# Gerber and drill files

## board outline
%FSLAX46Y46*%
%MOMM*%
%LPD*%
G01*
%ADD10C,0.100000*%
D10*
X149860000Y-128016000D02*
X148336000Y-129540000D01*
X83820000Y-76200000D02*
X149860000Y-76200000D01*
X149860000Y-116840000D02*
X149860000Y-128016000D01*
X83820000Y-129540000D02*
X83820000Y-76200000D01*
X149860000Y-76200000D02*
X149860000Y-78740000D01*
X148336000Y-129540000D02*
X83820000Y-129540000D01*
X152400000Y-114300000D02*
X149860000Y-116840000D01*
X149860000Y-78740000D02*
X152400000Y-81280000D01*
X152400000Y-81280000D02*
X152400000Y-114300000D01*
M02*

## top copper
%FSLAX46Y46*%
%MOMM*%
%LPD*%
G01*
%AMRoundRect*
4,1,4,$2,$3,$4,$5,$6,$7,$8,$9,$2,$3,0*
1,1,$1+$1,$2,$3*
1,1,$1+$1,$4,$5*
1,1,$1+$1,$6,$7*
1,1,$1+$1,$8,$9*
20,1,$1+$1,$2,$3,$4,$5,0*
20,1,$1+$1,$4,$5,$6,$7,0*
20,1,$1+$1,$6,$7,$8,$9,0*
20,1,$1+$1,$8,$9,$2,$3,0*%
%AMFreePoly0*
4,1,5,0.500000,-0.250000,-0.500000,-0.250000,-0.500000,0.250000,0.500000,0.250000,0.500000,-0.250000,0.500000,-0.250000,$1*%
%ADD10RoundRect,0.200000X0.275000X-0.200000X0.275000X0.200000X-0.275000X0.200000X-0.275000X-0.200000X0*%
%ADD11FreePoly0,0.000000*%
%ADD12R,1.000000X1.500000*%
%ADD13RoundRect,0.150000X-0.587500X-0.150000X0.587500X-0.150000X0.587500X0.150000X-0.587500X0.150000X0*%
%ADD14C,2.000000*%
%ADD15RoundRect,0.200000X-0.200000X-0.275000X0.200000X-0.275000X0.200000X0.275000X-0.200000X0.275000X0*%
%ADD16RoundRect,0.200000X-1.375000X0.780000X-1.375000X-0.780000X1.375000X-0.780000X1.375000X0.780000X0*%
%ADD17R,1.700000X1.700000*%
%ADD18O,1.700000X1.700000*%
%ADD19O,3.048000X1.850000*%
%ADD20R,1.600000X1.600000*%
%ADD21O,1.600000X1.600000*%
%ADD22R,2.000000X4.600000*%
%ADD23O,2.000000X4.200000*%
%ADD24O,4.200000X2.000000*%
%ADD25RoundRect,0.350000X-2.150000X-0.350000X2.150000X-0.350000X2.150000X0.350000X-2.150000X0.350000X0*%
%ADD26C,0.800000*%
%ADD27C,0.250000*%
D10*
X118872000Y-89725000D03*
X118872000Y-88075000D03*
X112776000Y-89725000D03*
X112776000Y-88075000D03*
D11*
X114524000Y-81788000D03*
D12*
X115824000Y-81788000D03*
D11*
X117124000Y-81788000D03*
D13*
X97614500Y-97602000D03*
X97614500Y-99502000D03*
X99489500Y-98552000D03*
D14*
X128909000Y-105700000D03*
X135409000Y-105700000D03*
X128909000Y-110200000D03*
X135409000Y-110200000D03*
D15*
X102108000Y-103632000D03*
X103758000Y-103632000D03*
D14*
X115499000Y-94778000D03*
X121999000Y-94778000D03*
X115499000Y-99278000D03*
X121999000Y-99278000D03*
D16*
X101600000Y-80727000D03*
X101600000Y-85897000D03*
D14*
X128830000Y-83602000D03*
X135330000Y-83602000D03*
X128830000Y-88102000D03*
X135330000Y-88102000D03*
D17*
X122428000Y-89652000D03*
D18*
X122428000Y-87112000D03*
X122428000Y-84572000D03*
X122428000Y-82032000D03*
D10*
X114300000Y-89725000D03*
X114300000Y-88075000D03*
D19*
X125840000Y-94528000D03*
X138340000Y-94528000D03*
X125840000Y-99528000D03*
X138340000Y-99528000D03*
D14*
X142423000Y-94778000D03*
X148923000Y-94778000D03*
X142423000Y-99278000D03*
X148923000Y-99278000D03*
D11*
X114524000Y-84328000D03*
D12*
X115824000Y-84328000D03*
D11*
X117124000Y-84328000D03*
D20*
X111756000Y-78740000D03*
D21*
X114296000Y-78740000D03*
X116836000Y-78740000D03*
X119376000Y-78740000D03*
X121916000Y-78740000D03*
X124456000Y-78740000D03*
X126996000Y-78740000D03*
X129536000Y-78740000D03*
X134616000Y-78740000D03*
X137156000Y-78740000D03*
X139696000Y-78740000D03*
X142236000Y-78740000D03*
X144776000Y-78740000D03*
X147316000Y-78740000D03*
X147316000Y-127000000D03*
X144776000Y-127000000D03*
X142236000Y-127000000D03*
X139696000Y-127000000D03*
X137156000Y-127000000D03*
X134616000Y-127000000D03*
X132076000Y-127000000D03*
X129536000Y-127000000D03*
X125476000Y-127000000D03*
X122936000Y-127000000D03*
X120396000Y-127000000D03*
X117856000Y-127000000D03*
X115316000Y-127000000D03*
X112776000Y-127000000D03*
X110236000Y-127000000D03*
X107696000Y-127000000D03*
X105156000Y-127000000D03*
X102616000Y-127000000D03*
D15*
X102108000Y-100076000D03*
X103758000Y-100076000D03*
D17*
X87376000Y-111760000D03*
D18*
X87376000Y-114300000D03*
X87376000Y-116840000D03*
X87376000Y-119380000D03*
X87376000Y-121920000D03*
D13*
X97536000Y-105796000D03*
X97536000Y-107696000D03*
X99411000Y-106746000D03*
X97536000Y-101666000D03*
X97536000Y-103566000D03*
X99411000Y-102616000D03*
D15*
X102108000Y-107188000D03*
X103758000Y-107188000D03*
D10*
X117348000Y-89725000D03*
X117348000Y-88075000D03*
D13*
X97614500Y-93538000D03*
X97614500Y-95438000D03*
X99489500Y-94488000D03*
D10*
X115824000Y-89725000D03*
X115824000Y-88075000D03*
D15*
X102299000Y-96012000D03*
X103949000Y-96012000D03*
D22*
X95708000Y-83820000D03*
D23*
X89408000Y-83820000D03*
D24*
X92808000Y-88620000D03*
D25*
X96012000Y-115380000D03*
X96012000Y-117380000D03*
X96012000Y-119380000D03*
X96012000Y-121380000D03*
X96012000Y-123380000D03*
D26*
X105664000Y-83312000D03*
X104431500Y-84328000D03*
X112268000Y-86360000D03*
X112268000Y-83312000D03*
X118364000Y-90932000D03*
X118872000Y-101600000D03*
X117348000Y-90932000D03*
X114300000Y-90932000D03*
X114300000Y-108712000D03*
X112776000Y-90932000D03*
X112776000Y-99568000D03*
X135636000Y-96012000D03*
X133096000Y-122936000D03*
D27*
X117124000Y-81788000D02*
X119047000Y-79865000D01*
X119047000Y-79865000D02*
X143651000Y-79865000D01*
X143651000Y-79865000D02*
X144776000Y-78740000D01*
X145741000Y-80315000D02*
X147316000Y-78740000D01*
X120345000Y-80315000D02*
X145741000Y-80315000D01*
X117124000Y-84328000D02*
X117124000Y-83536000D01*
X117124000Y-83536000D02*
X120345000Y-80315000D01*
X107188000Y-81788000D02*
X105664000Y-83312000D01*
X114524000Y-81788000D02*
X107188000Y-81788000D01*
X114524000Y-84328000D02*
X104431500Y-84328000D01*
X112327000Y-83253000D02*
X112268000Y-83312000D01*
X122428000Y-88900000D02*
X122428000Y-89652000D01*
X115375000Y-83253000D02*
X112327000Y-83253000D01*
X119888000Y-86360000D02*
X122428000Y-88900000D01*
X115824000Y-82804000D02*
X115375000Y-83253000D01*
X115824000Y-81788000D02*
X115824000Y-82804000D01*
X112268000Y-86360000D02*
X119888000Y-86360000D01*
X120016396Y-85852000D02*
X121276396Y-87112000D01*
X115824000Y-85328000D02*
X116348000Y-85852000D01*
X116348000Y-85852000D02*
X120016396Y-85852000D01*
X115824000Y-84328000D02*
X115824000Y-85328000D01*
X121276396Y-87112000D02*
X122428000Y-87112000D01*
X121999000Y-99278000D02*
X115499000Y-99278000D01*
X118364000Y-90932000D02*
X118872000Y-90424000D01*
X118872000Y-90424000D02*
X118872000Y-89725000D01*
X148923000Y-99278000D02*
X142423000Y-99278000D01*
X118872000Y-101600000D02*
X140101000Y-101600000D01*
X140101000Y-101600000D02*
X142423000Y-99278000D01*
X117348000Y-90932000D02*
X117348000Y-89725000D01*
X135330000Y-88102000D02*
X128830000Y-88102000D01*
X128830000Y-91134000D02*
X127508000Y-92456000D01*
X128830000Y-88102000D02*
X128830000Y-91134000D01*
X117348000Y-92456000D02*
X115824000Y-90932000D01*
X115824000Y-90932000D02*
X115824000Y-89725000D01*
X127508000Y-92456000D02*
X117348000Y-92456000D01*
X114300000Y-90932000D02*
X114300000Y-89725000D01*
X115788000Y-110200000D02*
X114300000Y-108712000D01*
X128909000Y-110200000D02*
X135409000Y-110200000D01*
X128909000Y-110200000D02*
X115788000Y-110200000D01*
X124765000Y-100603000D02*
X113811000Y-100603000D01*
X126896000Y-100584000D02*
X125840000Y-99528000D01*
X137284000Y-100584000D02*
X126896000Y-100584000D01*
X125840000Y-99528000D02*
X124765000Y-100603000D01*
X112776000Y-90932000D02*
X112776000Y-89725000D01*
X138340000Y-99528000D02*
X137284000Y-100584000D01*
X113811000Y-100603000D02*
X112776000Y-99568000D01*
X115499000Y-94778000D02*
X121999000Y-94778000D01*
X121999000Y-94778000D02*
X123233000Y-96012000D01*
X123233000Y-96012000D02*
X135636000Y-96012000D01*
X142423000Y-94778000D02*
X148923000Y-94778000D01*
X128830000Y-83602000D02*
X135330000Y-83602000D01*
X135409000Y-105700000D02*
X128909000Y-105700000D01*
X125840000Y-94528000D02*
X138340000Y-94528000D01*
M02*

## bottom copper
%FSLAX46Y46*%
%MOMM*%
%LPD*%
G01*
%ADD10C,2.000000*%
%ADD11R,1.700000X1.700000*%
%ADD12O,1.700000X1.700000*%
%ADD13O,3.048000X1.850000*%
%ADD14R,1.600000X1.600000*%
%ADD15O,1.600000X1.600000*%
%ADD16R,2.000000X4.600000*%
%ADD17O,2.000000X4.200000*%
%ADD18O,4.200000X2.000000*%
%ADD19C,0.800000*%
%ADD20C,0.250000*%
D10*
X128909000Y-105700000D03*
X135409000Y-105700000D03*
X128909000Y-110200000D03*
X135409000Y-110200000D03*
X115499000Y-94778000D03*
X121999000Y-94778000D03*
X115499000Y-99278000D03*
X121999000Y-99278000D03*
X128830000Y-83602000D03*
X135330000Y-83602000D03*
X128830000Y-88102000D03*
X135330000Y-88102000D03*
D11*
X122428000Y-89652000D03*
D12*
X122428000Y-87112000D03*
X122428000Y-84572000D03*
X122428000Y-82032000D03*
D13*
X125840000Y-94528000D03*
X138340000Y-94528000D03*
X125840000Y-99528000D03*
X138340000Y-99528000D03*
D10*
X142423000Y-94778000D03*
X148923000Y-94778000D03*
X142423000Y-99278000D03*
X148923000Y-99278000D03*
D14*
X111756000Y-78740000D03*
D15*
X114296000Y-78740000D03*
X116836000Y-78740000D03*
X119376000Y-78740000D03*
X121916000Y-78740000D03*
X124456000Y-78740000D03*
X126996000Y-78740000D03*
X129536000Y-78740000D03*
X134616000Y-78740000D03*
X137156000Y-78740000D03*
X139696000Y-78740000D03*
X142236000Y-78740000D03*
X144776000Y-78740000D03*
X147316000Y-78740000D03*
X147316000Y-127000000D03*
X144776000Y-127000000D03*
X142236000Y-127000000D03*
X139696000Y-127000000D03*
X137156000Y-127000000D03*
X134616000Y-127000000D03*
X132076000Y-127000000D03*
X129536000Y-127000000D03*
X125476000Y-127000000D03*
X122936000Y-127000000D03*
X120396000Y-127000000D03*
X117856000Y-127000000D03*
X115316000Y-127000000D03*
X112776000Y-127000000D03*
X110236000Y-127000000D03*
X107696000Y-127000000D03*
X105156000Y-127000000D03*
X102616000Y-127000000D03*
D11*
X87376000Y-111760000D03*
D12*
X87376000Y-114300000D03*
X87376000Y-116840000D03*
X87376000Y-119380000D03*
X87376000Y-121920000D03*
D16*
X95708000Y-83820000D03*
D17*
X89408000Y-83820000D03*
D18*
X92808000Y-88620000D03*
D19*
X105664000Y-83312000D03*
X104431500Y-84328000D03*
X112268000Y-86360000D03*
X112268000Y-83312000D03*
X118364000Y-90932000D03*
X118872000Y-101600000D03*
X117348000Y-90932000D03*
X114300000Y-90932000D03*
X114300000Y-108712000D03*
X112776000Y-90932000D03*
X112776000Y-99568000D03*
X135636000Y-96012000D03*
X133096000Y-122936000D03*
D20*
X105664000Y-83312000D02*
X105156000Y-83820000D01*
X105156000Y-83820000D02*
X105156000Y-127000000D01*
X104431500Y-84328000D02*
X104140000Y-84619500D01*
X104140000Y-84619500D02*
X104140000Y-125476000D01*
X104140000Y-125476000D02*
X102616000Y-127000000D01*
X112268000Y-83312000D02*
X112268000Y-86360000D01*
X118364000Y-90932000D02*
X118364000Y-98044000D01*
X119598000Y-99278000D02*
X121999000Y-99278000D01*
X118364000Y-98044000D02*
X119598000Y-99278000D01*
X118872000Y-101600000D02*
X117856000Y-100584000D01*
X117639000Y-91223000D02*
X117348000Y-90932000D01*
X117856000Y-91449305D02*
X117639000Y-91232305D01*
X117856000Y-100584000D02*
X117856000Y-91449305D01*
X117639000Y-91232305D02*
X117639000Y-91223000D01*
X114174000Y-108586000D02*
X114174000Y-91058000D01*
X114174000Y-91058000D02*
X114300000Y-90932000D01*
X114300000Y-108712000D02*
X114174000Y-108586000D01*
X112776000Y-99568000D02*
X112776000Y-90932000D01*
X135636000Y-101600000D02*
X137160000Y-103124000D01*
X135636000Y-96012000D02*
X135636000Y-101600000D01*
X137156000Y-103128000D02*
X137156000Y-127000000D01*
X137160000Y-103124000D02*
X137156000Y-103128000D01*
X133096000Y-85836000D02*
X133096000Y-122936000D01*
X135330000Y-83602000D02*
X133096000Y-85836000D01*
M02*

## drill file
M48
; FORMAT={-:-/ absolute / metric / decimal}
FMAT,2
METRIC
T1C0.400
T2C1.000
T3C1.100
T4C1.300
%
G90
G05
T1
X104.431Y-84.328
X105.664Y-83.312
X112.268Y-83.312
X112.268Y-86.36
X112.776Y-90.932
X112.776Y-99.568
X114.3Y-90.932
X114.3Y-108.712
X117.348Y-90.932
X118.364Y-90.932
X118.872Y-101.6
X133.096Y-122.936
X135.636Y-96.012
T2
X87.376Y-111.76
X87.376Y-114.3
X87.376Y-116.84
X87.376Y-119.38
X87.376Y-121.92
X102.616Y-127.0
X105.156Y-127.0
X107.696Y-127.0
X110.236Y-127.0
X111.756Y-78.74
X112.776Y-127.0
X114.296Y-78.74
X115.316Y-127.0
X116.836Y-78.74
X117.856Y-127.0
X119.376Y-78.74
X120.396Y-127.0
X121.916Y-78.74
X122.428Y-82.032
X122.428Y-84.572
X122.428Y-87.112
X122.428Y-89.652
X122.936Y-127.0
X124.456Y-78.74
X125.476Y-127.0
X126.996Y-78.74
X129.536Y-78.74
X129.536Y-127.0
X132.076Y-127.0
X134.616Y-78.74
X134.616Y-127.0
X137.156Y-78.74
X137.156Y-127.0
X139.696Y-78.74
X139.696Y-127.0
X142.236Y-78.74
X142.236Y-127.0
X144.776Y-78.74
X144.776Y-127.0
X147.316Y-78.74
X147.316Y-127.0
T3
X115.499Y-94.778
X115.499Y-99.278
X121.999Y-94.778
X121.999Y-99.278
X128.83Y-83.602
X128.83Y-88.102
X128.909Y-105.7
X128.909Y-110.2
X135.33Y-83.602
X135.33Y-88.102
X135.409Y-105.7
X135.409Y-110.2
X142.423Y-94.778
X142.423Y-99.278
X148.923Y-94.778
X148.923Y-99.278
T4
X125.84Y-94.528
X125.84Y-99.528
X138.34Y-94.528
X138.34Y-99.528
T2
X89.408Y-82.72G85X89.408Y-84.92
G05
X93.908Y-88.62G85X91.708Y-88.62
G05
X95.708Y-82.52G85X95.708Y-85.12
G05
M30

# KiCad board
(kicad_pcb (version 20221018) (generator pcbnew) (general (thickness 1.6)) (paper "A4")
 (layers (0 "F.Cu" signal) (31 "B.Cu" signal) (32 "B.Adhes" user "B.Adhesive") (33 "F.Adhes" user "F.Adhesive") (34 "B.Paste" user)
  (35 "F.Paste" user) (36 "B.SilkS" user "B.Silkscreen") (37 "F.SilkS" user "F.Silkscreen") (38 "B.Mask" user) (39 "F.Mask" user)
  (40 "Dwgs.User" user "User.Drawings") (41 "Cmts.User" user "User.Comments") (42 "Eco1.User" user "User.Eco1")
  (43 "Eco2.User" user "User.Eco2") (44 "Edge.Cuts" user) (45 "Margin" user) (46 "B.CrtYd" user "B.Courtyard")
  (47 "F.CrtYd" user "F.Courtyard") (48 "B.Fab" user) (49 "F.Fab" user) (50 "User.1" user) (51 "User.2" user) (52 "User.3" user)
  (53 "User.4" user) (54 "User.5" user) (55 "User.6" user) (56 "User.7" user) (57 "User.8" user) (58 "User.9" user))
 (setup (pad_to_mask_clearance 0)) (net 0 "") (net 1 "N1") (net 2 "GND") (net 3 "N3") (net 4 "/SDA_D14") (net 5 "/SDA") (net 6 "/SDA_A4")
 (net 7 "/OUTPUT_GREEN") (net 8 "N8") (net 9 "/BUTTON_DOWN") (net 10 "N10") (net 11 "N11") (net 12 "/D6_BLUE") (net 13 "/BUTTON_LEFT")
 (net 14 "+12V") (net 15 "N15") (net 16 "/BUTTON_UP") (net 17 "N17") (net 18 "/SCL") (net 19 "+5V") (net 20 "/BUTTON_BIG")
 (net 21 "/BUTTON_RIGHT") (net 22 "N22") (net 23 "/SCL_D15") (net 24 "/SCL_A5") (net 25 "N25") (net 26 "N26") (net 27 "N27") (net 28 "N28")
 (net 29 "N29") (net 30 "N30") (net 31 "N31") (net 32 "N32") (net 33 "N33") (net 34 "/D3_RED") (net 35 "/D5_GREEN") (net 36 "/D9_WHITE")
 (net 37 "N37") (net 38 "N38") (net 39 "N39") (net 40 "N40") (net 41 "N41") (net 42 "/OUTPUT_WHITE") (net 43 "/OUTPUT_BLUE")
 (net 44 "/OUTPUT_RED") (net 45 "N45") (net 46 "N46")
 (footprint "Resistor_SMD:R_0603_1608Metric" (layer "F.Cu") (at 118.872 88.9 90)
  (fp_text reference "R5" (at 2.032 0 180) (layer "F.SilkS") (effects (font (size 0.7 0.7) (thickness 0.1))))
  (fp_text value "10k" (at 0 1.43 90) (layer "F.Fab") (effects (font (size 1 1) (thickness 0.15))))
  (pad "1" smd roundrect (at -0.825 0 90) (size 0.8 0.95) (layers "F.Cu" "F.Paste" "F.Mask") (roundrect_rratio 0.25) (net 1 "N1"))
  (pad "2" smd roundrect (at 0.825 0 90) (size 0.8 0.95) (layers "F.Cu" "F.Paste" "F.Mask") (roundrect_rratio 0.25) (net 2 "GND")))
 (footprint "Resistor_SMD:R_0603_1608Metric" (layer "F.Cu") (at 112.776 88.9 90)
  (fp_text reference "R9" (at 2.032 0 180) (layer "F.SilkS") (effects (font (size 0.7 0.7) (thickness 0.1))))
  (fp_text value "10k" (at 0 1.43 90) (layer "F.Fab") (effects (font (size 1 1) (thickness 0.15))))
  (pad "1" smd roundrect (at -0.825 0 90) (size 0.8 0.95) (layers "F.Cu" "F.Paste" "F.Mask") (roundrect_rratio 0.25) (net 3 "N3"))
  (pad "2" smd roundrect (at 0.825 0 90) (size 0.8 0.95) (layers "F.Cu" "F.Paste" "F.Mask") (roundrect_rratio 0.25) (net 2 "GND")))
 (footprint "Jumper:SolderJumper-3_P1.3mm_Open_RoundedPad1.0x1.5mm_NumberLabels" (layer "F.Cu") (at 115.824 81.788)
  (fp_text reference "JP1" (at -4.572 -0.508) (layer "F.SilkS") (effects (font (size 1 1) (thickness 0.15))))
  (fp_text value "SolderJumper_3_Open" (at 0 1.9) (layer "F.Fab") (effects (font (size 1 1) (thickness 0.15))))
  (pad "1" smd custom (at -1.3 0) (size 1 0.5) (layers "F.Cu" "F.Mask") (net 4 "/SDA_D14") (zone_connect 2) (thermal_bridge_angle 45)
   (options (clearance outline) (anchor rect)) (primitives))
  (pad "2" smd rect (at 0 0) (size 1 1.5) (layers "F.Cu" "F.Mask") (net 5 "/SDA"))
  (pad "3" smd custom (at 1.3 0) (size 1 0.5) (layers "F.Cu" "F.Mask") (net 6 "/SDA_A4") (zone_connect 2) (thermal_bridge_angle 45)
   (options (clearance outline) (anchor rect)) (primitives)))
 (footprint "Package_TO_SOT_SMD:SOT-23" (layer "F.Cu") (at 98.552 98.552)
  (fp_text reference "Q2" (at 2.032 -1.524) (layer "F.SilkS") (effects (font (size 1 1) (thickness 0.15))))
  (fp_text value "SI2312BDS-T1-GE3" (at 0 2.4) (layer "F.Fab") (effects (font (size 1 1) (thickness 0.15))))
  (pad "1" smd roundrect (at -0.9375 -0.95) (size 1.475 0.6) (layers "F.Cu" "F.Paste" "F.Mask") (roundrect_rratio 0.25)
   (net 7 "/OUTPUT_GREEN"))
  (pad "2" smd roundrect (at -0.9375 0.95) (size 1.475 0.6) (layers "F.Cu" "F.Paste" "F.Mask") (roundrect_rratio 0.25) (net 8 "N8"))
  (pad "3" smd roundrect (at 0.9375 0) (size 1.475 0.6) (layers "F.Cu" "F.Paste" "F.Mask") (roundrect_rratio 0.25) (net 2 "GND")))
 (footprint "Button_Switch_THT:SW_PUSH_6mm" (layer "F.Cu") (at 128.909 105.7)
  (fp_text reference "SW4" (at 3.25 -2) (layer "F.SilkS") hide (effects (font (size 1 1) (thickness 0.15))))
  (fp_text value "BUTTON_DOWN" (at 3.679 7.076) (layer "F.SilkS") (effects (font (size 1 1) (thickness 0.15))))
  (pad "1" thru_hole circle (at 0 0 90) (size 2 2) (drill 1.1) (layers "*.Cu" "*.Mask") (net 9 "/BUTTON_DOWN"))
  (pad "1" thru_hole circle (at 6.5 0 90) (size 2 2) (drill 1.1) (layers "*.Cu" "*.Mask") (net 9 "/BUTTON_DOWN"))
  (pad "2" thru_hole circle (at 0 4.5 90) (size 2 2) (drill 1.1) (layers "*.Cu" "*.Mask") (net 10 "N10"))
  (pad "2" thru_hole circle (at 6.5 4.5 90) (size 2 2) (drill 1.1) (layers "*.Cu" "*.Mask") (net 10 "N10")))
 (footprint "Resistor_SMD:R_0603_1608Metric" (layer "F.Cu") (at 102.933 103.632)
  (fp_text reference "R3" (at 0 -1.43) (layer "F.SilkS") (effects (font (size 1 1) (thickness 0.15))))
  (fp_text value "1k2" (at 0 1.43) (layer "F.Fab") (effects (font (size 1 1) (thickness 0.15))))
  (pad "1" smd roundrect (at -0.825 0) (size 0.8 0.95) (layers "F.Cu" "F.Paste" "F.Mask") (roundrect_rratio 0.25) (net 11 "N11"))
  (pad "2" smd roundrect (at 0.825 0) (size 0.8 0.95) (layers "F.Cu" "F.Paste" "F.Mask") (roundrect_rratio 0.25) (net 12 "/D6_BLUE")))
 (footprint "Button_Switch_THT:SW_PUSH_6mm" (layer "F.Cu") (at 115.499 94.778)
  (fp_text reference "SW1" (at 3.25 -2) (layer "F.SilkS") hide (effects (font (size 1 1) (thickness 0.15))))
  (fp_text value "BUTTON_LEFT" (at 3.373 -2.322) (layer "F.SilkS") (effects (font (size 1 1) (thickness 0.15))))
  (pad "1" thru_hole circle (at 0 0 90) (size 2 2) (drill 1.1) (layers "*.Cu" "*.Mask") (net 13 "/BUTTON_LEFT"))
  (pad "1" thru_hole circle (at 6.5 0 90) (size 2 2) (drill 1.1) (layers "*.Cu" "*.Mask") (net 13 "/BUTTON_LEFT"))
  (pad "2" thru_hole circle (at 0 4.5 90) (size 2 2) (drill 1.1) (layers "*.Cu" "*.Mask") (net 1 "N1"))
  (pad "2" thru_hole circle (at 6.5 4.5 90) (size 2 2) (drill 1.1) (layers "*.Cu" "*.Mask") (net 1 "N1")))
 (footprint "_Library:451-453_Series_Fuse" (layer "F.Cu") (at 101.6 83.312 -90)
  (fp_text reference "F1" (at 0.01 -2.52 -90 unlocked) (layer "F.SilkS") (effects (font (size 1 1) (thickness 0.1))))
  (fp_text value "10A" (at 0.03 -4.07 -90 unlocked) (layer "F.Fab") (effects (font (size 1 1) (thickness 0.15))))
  (pad "1" smd roundrect (at -2.585 0 270) (size 1.96 3.15) (layers "F.Cu" "F.Paste" "F.Mask") (roundrect_rratio 0.1020408163)
   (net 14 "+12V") (thermal_bridge_angle 45))
  (pad "2" smd roundrect (at 2.585 0 270) (size 1.96 3.15) (layers "F.Cu" "F.Paste" "F.Mask") (roundrect_rratio 0.1020408163) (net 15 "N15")
   (thermal_bridge_angle 45)))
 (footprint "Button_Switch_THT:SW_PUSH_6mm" (layer "F.Cu") (at 128.83 83.602)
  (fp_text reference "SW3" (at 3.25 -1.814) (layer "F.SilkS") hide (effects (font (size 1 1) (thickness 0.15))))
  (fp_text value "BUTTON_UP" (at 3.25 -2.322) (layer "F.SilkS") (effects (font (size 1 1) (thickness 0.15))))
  (pad "1" thru_hole circle (at 0 0 90) (size 2 2) (drill 1.1) (layers "*.Cu" "*.Mask") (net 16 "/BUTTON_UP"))
  (pad "1" thru_hole circle (at 6.5 0 90) (size 2 2) (drill 1.1) (layers "*.Cu" "*.Mask") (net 16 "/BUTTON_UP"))
  (pad "2" thru_hole circle (at 0 4.5 90) (size 2 2) (drill 1.1) (layers "*.Cu" "*.Mask") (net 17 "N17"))
  (pad "2" thru_hole circle (at 6.5 4.5 90) (size 2 2) (drill 1.1) (layers "*.Cu" "*.Mask") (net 17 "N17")))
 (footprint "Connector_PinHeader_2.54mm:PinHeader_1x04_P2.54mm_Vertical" (layer "F.Cu") (at 122.428 89.652 180)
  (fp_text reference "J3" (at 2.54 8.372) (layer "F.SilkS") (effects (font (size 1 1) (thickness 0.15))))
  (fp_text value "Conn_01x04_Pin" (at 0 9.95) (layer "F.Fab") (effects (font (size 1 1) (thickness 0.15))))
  (pad "1" thru_hole rect (at 0 0 180) (size 1.7 1.7) (drill 1) (layers "*.Cu" "*.Mask") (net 5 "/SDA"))
  (pad "2" thru_hole oval (at 0 2.54 180) (size 1.7 1.7) (drill 1) (layers "*.Cu" "*.Mask") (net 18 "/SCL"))
  (pad "3" thru_hole oval (at 0 5.08 180) (size 1.7 1.7) (drill 1) (layers "*.Cu" "*.Mask") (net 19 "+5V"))
  (pad "4" thru_hole oval (at 0 7.62 180) (size 1.7 1.7) (drill 1) (layers "*.Cu" "*.Mask") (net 2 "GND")))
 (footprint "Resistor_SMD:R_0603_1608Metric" (layer "F.Cu") (at 114.3 88.9 90)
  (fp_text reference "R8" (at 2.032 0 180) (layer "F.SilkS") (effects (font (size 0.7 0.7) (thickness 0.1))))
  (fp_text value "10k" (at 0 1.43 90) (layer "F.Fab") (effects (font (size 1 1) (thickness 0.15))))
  (pad "1" smd roundrect (at -0.825 0 90) (size 0.8 0.95) (layers "F.Cu" "F.Paste" "F.Mask") (roundrect_rratio 0.25) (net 10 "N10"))
  (pad "2" smd roundrect (at 0.825 0 90) (size 0.8 0.95) (layers "F.Cu" "F.Paste" "F.Mask") (roundrect_rratio 0.25) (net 2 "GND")))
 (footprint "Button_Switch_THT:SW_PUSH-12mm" (layer "F.Cu") (at 125.84 94.528)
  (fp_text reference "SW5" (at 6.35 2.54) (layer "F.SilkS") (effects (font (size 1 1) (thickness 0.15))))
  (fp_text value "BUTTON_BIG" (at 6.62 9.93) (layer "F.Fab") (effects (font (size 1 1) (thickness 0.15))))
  (pad "1" thru_hole oval (at 0 0) (size 3.048 1.85) (drill 1.3) (layers "*.Cu" "*.Mask") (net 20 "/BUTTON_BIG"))
  (pad "1" thru_hole oval (at 12.5 0) (size 3.048 1.85) (drill 1.3) (layers "*.Cu" "*.Mask") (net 20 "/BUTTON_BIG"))
  (pad "2" thru_hole oval (at 0 5) (size 3.048 1.85) (drill 1.3) (layers "*.Cu" "*.Mask") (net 3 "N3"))
  (pad "2" thru_hole oval (at 12.5 5) (size 3.048 1.85) (drill 1.3) (layers "*.Cu" "*.Mask") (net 3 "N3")))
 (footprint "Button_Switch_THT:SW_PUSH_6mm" (layer "F.Cu") (at 142.423 94.778)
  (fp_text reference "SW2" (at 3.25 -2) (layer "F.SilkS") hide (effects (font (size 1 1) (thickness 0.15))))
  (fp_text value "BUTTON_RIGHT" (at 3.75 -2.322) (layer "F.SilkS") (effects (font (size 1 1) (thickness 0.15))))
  (pad "1" thru_hole circle (at 0 0 90) (size 2 2) (drill 1.1) (layers "*.Cu" "*.Mask") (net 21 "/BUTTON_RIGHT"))
  (pad "1" thru_hole circle (at 6.5 0 90) (size 2 2) (drill 1.1) (layers "*.Cu" "*.Mask") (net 21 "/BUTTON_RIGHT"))
  (pad "2" thru_hole circle (at 0 4.5 90) (size 2 2) (drill 1.1) (layers "*.Cu" "*.Mask") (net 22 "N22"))
  (pad "2" thru_hole circle (at 6.5 4.5 90) (size 2 2) (drill 1.1) (layers "*.Cu" "*.Mask") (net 22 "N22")))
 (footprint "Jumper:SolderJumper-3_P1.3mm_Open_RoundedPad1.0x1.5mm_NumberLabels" (layer "F.Cu") (at 115.824 84.328)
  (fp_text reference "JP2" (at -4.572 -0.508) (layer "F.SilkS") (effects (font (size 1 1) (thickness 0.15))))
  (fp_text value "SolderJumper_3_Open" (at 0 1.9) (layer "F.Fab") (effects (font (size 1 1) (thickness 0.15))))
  (pad "1" smd custom (at -1.3 0) (size 1 0.5) (layers "F.Cu" "F.Mask") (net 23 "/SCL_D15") (zone_connect 2) (thermal_bridge_angle 45)
   (options (clearance outline) (anchor rect)) (primitives))
  (pad "2" smd rect (at 0 0) (size 1 1.5) (layers "F.Cu" "F.Mask") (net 18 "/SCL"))
  (pad "3" smd custom (at 1.3 0) (size 1 0.5) (layers "F.Cu" "F.Mask") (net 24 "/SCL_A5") (zone_connect 2) (thermal_bridge_angle 45)
   (options (clearance outline) (anchor rect)) (primitives)))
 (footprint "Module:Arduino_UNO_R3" (layer "F.Cu") (at 111.756 78.74)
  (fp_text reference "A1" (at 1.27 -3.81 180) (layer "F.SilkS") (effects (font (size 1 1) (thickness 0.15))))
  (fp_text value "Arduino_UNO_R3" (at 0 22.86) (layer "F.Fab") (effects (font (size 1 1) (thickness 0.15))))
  (pad "1" thru_hole rect (at 0 0 90) (size 1.6 1.6) (drill 1) (layers "*.Cu" "*.Mask") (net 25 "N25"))
  (pad "2" thru_hole oval (at 2.54 0 90) (size 1.6 1.6) (drill 1) (layers "*.Cu" "*.Mask") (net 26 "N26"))
  (pad "3" thru_hole oval (at 5.08 0 90) (size 1.6 1.6) (drill 1) (layers "*.Cu" "*.Mask") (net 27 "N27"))
  (pad "4" thru_hole oval (at 7.62 0 90) (size 1.6 1.6) (drill 1) (layers "*.Cu" "*.Mask") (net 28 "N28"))
  (pad "5" thru_hole oval (at 10.16 0 90) (size 1.6 1.6) (drill 1) (layers "*.Cu" "*.Mask") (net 19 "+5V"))
  (pad "6" thru_hole oval (at 12.7 0 90) (size 1.6 1.6) (drill 1) (layers "*.Cu" "*.Mask") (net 2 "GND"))
  (pad "7" thru_hole oval (at 15.24 0 90) (size 1.6 1.6) (drill 1) (layers "*.Cu" "*.Mask") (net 2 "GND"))
  (pad "8" thru_hole oval (at 17.78 0 90) (size 1.6 1.6) (drill 1) (layers "*.Cu" "*.Mask") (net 14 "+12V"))
  (pad "9" thru_hole oval (at 22.86 0 90) (size 1.6 1.6) (drill 1) (layers "*.Cu" "*.Mask") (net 9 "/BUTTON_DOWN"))
  (pad "10" thru_hole oval (at 25.4 0 90) (size 1.6 1.6) (drill 1) (layers "*.Cu" "*.Mask") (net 20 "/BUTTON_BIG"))
  (pad "11" thru_hole oval (at 27.94 0 90) (size 1.6 1.6) (drill 1) (layers "*.Cu" "*.Mask") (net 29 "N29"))
  (pad "12" thru_hole oval (at 30.48 0 90) (size 1.6 1.6) (drill 1) (layers "*.Cu" "*.Mask") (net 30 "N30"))
  (pad "13" thru_hole oval (at 33.02 0 90) (size 1.6 1.6) (drill 1) (layers "*.Cu" "*.Mask") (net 6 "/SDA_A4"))
  (pad "14" thru_hole oval (at 35.56 0 90) (size 1.6 1.6) (drill 1) (layers "*.Cu" "*.Mask") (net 24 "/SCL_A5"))
  (pad "15" thru_hole oval (at 35.56 48.26 90) (size 1.6 1.6) (drill 1) (layers "*.Cu" "*.Mask") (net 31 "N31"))
  (pad "16" thru_hole oval (at 33.02 48.26 90) (size 1.6 1.6) (drill 1) (layers "*.Cu" "*.Mask") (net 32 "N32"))
  (pad "17" thru_hole oval (at 30.48 48.26 90) (size 1.6 1.6) (drill 1) (layers "*.Cu" "*.Mask") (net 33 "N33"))
  (pad "18" thru_hole oval (at 27.94 48.26 90) (size 1.6 1.6) (drill 1) (layers "*.Cu" "*.Mask") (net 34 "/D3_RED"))
  (pad "19" thru_hole oval (at 25.4 48.26 90) (size 1.6 1.6) (drill 1) (layers "*.Cu" "*.Mask") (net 13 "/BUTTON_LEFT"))
  (pad "20" thru_hole oval (at 22.86 48.26 90) (size 1.6 1.6) (drill 1) (layers "*.Cu" "*.Mask") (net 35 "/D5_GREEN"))
  (pad "21" thru_hole oval (at 20.32 48.26 90) (size 1.6 1.6) (drill 1) (layers "*.Cu" "*.Mask") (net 12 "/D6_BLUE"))
  (pad "22" thru_hole oval (at 17.78 48.26 90) (size 1.6 1.6) (drill 1) (layers "*.Cu" "*.Mask") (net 21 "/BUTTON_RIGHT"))
  (pad "23" thru_hole oval (at 13.72 48.26 90) (size 1.6 1.6) (drill 1) (layers "*.Cu" "*.Mask") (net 16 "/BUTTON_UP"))
  (pad "24" thru_hole oval (at 11.18 48.26 90) (size 1.6 1.6) (drill 1) (layers "*.Cu" "*.Mask") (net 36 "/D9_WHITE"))
  (pad "25" thru_hole oval (at 8.64 48.26 90) (size 1.6 1.6) (drill 1) (layers "*.Cu" "*.Mask") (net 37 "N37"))
  (pad "26" thru_hole oval (at 6.1 48.26 90) (size 1.6 1.6) (drill 1) (layers "*.Cu" "*.Mask") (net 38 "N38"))
  (pad "27" thru_hole oval (at 3.56 48.26 90) (size 1.6 1.6) (drill 1) (layers "*.Cu" "*.Mask") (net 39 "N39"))
  (pad "28" thru_hole oval (at 1.02 48.26 90) (size 1.6 1.6) (drill 1) (layers "*.Cu" "*.Mask") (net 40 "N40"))
  (pad "29" thru_hole oval (at -1.52 48.26 90) (size 1.6 1.6) (drill 1) (layers "*.Cu" "*.Mask") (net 2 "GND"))
  (pad "30" thru_hole oval (at -4.06 48.26 90) (size 1.6 1.6) (drill 1) (layers "*.Cu" "*.Mask") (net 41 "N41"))
  (pad "31" thru_hole oval (at -6.6 48.26 90) (size 1.6 1.6) (drill 1) (layers "*.Cu" "*.Mask") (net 4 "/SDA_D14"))
  (pad "32" thru_hole oval (at -9.14 48.26 90) (size 1.6 1.6) (drill 1) (layers "*.Cu" "*.Mask") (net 23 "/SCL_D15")))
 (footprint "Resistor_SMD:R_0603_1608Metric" (layer "F.Cu") (at 102.933 100.076)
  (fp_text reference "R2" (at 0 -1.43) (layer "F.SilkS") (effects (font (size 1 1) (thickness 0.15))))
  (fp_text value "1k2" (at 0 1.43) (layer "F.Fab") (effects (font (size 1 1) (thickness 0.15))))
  (pad "1" smd roundrect (at -0.825 0) (size 0.8 0.95) (layers "F.Cu" "F.Paste" "F.Mask") (roundrect_rratio 0.25) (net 8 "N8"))
  (pad "2" smd roundrect (at 0.825 0) (size 0.8 0.95) (layers "F.Cu" "F.Paste" "F.Mask") (roundrect_rratio 0.25) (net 35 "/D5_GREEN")))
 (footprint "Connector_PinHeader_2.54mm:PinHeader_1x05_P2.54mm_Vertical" (layer "F.Cu") (at 87.376 111.76)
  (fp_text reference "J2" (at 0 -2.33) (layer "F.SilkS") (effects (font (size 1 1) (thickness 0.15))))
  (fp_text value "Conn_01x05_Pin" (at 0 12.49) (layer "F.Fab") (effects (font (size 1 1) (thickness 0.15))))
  (pad "1" thru_hole rect (at 0 0) (size 1.7 1.7) (drill 1) (layers "*.Cu" "*.Mask") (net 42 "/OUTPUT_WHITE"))
  (pad "2" thru_hole oval (at 0 2.54) (size 1.7 1.7) (drill 1) (layers "*.Cu" "*.Mask") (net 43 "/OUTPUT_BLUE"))
  (pad "3" thru_hole oval (at 0 5.08) (size 1.7 1.7) (drill 1) (layers "*.Cu" "*.Mask") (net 7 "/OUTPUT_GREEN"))
  (pad "4" thru_hole oval (at 0 7.62) (size 1.7 1.7) (drill 1) (layers "*.Cu" "*.Mask") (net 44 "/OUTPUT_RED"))
  (pad "5" thru_hole oval (at 0 10.16) (size 1.7 1.7) (drill 1) (layers "*.Cu" "*.Mask") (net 14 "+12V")))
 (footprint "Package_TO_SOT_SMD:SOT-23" (layer "F.Cu") (at 98.4735 106.746)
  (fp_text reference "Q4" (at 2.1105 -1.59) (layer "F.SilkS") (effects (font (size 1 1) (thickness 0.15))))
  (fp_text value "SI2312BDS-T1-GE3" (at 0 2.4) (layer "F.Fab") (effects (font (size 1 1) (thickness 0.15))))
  (pad "1" smd roundrect (at -0.9375 -0.95) (size 1.475 0.6) (layers "F.Cu" "F.Paste" "F.Mask") (roundrect_rratio 0.25)
   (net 42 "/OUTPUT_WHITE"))
  (pad "2" smd roundrect (at -0.9375 0.95) (size 1.475 0.6) (layers "F.Cu" "F.Paste" "F.Mask") (roundrect_rratio 0.25) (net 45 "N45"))
  (pad "3" smd roundrect (at 0.9375 0) (size 1.475 0.6) (layers "F.Cu" "F.Paste" "F.Mask") (roundrect_rratio 0.25) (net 2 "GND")))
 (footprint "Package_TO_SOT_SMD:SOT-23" (layer "F.Cu") (at 98.4735 102.616)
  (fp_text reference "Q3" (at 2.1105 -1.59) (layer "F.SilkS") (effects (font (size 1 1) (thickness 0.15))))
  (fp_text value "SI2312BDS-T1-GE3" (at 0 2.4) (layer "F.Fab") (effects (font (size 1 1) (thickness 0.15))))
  (pad "1" smd roundrect (at -0.9375 -0.95) (size 1.475 0.6) (layers "F.Cu" "F.Paste" "F.Mask") (roundrect_rratio 0.25)
   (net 43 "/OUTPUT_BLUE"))
  (pad "2" smd roundrect (at -0.9375 0.95) (size 1.475 0.6) (layers "F.Cu" "F.Paste" "F.Mask") (roundrect_rratio 0.25) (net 11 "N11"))
  (pad "3" smd roundrect (at 0.9375 0) (size 1.475 0.6) (layers "F.Cu" "F.Paste" "F.Mask") (roundrect_rratio 0.25) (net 2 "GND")))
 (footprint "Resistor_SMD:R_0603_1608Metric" (layer "F.Cu") (at 102.933 107.188)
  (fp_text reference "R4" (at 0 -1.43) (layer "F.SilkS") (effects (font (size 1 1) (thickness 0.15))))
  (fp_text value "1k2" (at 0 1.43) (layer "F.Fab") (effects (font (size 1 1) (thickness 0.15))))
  (pad "1" smd roundrect (at -0.825 0) (size 0.8 0.95) (layers "F.Cu" "F.Paste" "F.Mask") (roundrect_rratio 0.25) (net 45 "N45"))
  (pad "2" smd roundrect (at 0.825 0) (size 0.8 0.95) (layers "F.Cu" "F.Paste" "F.Mask") (roundrect_rratio 0.25) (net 36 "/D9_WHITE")))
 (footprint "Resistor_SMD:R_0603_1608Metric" (layer "F.Cu") (at 117.348 88.9 90)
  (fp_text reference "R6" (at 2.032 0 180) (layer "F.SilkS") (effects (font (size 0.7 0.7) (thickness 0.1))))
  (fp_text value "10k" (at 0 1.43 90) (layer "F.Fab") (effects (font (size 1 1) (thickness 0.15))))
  (pad "1" smd roundrect (at -0.825 0 90) (size 0.8 0.95) (layers "F.Cu" "F.Paste" "F.Mask") (roundrect_rratio 0.25) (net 22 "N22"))
  (pad "2" smd roundrect (at 0.825 0 90) (size 0.8 0.95) (layers "F.Cu" "F.Paste" "F.Mask") (roundrect_rratio 0.25) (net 2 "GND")))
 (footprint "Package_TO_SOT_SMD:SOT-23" (layer "F.Cu") (at 98.552 94.488)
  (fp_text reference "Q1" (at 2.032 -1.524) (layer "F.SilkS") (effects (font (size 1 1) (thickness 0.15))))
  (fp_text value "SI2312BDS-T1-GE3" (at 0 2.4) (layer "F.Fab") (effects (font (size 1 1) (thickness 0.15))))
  (pad "1" smd roundrect (at -0.9375 -0.95) (size 1.475 0.6) (layers "F.Cu" "F.Paste" "F.Mask") (roundrect_rratio 0.25)
   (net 44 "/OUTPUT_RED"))
  (pad "2" smd roundrect (at -0.9375 0.95) (size 1.475 0.6) (layers "F.Cu" "F.Paste" "F.Mask") (roundrect_rratio 0.25) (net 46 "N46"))
  (pad "3" smd roundrect (at 0.9375 0) (size 1.475 0.6) (layers "F.Cu" "F.Paste" "F.Mask") (roundrect_rratio 0.25) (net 2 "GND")))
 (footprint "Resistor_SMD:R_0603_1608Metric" (layer "F.Cu") (at 115.824 88.9 90)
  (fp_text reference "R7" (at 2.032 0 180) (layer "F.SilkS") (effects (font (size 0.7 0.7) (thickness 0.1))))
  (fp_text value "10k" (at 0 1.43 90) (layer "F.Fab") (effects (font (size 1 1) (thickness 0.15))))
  (pad "1" smd roundrect (at -0.825 0 90) (size 0.8 0.95) (layers "F.Cu" "F.Paste" "F.Mask") (roundrect_rratio 0.25) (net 17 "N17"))
  (pad "2" smd roundrect (at 0.825 0 90) (size 0.8 0.95) (layers "F.Cu" "F.Paste" "F.Mask") (roundrect_rratio 0.25) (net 2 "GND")))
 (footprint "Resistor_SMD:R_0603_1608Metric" (layer "F.Cu") (at 103.124 96.012)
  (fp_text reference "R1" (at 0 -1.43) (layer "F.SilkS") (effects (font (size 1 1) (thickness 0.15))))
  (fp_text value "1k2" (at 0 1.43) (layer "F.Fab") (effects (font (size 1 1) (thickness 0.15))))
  (pad "1" smd roundrect (at -0.825 0) (size 0.8 0.95) (layers "F.Cu" "F.Paste" "F.Mask") (roundrect_rratio 0.25) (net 46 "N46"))
  (pad "2" smd roundrect (at 0.825 0) (size 0.8 0.95) (layers "F.Cu" "F.Paste" "F.Mask") (roundrect_rratio 0.25) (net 34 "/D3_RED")))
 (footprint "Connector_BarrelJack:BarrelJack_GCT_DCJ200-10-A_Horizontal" (layer "F.Cu") (at 95.708 83.82 -90)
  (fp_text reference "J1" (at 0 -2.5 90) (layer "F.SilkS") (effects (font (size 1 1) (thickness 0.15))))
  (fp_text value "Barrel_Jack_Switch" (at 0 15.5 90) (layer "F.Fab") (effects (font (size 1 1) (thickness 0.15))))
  (pad "1" thru_hole rect (at 0 0 270) (size 4.6 2) (drill oval 3.6 1) (layers "*.Cu" "*.Mask") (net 15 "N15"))
  (pad "2" thru_hole oval (at 0 6.3 270) (size 4.2 2) (drill oval 3.2 1) (layers "*.Cu" "*.Mask") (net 2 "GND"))
  (pad "3" thru_hole oval (at 4.8 2.9 270) (size 2 4.2) (drill oval 1 3.2) (layers "*.Cu" "*.Mask") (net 2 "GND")))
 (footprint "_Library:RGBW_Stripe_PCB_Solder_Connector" (layer "F.Cu") (at 96.012 119.38)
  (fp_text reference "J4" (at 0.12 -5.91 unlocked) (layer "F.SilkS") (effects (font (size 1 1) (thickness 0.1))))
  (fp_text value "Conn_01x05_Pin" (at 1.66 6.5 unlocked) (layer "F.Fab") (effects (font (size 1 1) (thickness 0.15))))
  (pad "1" smd roundrect (at 0 -4) (size 5 1.4) (layers "F.Cu" "F.Paste" "F.Mask") (roundrect_rratio 0.25) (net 42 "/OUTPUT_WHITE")
   (thermal_bridge_angle 45))
  (pad "2" smd roundrect (at 0 -2) (size 5 1.4) (layers "F.Cu" "F.Paste" "F.Mask") (roundrect_rratio 0.25) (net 43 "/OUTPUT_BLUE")
   (thermal_bridge_angle 45))
  (pad "3" smd roundrect (at 0 0) (size 5 1.4) (layers "F.Cu" "F.Paste" "F.Mask") (roundrect_rratio 0.25) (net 7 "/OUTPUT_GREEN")
   (thermal_bridge_angle 45))
  (pad "4" smd roundrect (at 0 2) (size 5 1.4) (layers "F.Cu" "F.Paste" "F.Mask") (roundrect_rratio 0.25) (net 44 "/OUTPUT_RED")
   (thermal_bridge_angle 45))
  (pad "5" smd roundrect (at 0 4) (size 5 1.4) (layers "F.Cu" "F.Paste" "F.Mask") (roundrect_rratio 0.25) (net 14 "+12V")
   (thermal_bridge_angle 45)))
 (gr_line (start 149.86 128.016) (end 148.336 129.54) (stroke (width 0.1) (type default)) (layer "Edge.Cuts"))
 (gr_line (start 83.82 76.2) (end 149.86 76.2) (stroke (width 0.1) (type default)) (layer "Edge.Cuts"))
 (gr_line (start 149.86 116.84) (end 149.86 128.016) (stroke (width 0.1) (type default)) (layer "Edge.Cuts"))
 (gr_line (start 83.82 129.54) (end 83.82 76.2) (stroke (width 0.1) (type default)) (layer "Edge.Cuts"))
 (gr_line (start 149.86 76.2) (end 149.86 78.74) (stroke (width 0.1) (type default)) (layer "Edge.Cuts"))
 (gr_line (start 148.336 129.54) (end 83.82 129.54) (stroke (width 0.1) (type default)) (layer "Edge.Cuts"))
 (gr_line (start 152.4 114.3) (end 149.86 116.84) (stroke (width 0.1) (type default)) (layer "Edge.Cuts"))
 (gr_line (start 149.86 78.74) (end 152.4 81.28) (stroke (width 0.1) (type default)) (layer "Edge.Cuts"))
 (gr_line (start 152.4 81.28) (end 152.4 114.3) (stroke (width 0.1) (type default)) (layer "Edge.Cuts"))
 (segment (start 117.124 81.788) (end 119.047 79.865) (width 0.25) (layer "F.Cu") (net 6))
 (segment (start 119.047 79.865) (end 143.651 79.865) (width 0.25) (layer "F.Cu") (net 6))
 (segment (start 143.651 79.865) (end 144.776 78.74) (width 0.25) (layer "F.Cu") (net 6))
 (segment (start 145.741 80.315) (end 147.316 78.74) (width 0.25) (layer "F.Cu") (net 24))
 (segment (start 120.345 80.315) (end 145.741 80.315) (width 0.25) (layer "F.Cu") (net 24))
 (segment (start 117.124 84.328) (end 117.124 83.536) (width 0.25) (layer "F.Cu") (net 24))
 (segment (start 117.124 83.536) (end 120.345 80.315) (width 0.25) (layer "F.Cu") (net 24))
 (segment (start 107.188 81.788) (end 105.664 83.312) (width 0.25) (layer "F.Cu") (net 4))
 (segment (start 114.524 81.788) (end 107.188 81.788) (width 0.25) (layer "F.Cu") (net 4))
 (via (at 105.664 83.312) (size 0.8) (drill 0.4) (layers "F.Cu" "B.Cu") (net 4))
 (segment (start 105.664 83.312) (end 105.156 83.82) (width 0.25) (layer "B.Cu") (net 4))
 (segment (start 105.156 83.82) (end 105.156 127) (width 0.25) (layer "B.Cu") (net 4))
 (segment (start 114.524 84.328) (end 104.4315 84.328) (width 0.25) (layer "F.Cu") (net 23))
 (via (at 104.4315 84.328) (size 0.8) (drill 0.4) (layers "F.Cu" "B.Cu") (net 23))
 (segment (start 104.4315 84.328) (end 104.14 84.6195) (width 0.25) (layer "B.Cu") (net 23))
 (segment (start 104.14 84.6195) (end 104.14 125.476) (width 0.25) (layer "B.Cu") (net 23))
 (segment (start 104.14 125.476) (end 102.616 127) (width 0.25) (layer "B.Cu") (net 23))
 (segment (start 112.327 83.253) (end 112.268 83.312) (width 0.25) (layer "F.Cu") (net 5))
 (segment (start 122.428 88.9) (end 122.428 89.652) (width 0.25) (layer "F.Cu") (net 5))
 (segment (start 115.375 83.253) (end 112.327 83.253) (width 0.25) (layer "F.Cu") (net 5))
 (segment (start 119.888 86.36) (end 122.428 88.9) (width 0.25) (layer "F.Cu") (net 5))
 (segment (start 115.824 82.804) (end 115.375 83.253) (width 0.25) (layer "F.Cu") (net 5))
 (segment (start 115.824 81.788) (end 115.824 82.804) (width 0.25) (layer "F.Cu") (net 5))
 (segment (start 112.268 86.36) (end 119.888 86.36) (width 0.25) (layer "F.Cu") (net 5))
 (via (at 112.268 86.36) (size 0.8) (drill 0.4) (layers "F.Cu" "B.Cu") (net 5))
 (via (at 112.268 83.312) (size 0.8) (drill 0.4) (layers "F.Cu" "B.Cu") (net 5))
 (segment (start 112.268 83.312) (end 112.268 86.36) (width 0.25) (layer "B.Cu") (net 5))
 (segment (start 120.016396 85.852) (end 121.276396 87.112) (width 0.25) (layer "F.Cu") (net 18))
 (segment (start 115.824 85.328) (end 116.348 85.852) (width 0.25) (layer "F.Cu") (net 18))
 (segment (start 116.348 85.852) (end 120.016396 85.852) (width 0.25) (layer "F.Cu") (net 18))
 (segment (start 115.824 84.328) (end 115.824 85.328) (width 0.25) (layer "F.Cu") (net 18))
 (segment (start 121.276396 87.112) (end 122.428 87.112) (width 0.25) (layer "F.Cu") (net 18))
 (segment (start 121.999 99.278) (end 115.499 99.278) (width 0.25) (layer "F.Cu") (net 1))
 (segment (start 118.364 90.932) (end 118.872 90.424) (width 0.25) (layer "F.Cu") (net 1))
 (segment (start 118.872 90.424) (end 118.872 89.725) (width 0.25) (layer "F.Cu") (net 1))
 (via (at 118.364 90.932) (size 0.8) (drill 0.4) (layers "F.Cu" "B.Cu") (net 1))
 (segment (start 118.364 90.932) (end 118.364 98.044) (width 0.25) (layer "B.Cu") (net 1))
 (segment (start 119.598 99.278) (end 121.999 99.278) (width 0.25) (layer "B.Cu") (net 1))
 (segment (start 118.364 98.044) (end 119.598 99.278) (width 0.25) (layer "B.Cu") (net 1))
 (segment (start 148.923 99.278) (end 142.423 99.278) (width 0.25) (layer "F.Cu") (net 22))
 (segment (start 118.872 101.6) (end 140.101 101.6) (width 0.25) (layer "F.Cu") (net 22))
 (segment (start 140.101 101.6) (end 142.423 99.278) (width 0.25) (layer "F.Cu") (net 22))
 (segment (start 117.348 90.932) (end 117.348 89.725) (width 0.25) (layer "F.Cu") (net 22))
 (via (at 118.872 101.6) (size 0.8) (drill 0.4) (layers "F.Cu" "B.Cu") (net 22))
 (via (at 117.348 90.932) (size 0.8) (drill 0.4) (layers "F.Cu" "B.Cu") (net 22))
 (segment (start 118.872 101.6) (end 117.856 100.584) (width 0.25) (layer "B.Cu") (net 22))
 (segment (start 117.639 91.223) (end 117.348 90.932) (width 0.25) (layer "B.Cu") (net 22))
 (segment (start 117.856 91.449305) (end 117.639 91.232305) (width 0.25) (layer "B.Cu") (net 22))
 (segment (start 117.856 100.584) (end 117.856 91.449305) (width 0.25) (layer "B.Cu") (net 22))
 (segment (start 117.639 91.232305) (end 117.639 91.223) (width 0.25) (layer "B.Cu") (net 22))
 (segment (start 135.33 88.102) (end 128.83 88.102) (width 0.25) (layer "F.Cu") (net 17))
 (segment (start 128.83 91.134) (end 127.508 92.456) (width 0.25) (layer "F.Cu") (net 17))
 (segment (start 128.83 88.102) (end 128.83 91.134) (width 0.25) (layer "F.Cu") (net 17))
 (segment (start 117.348 92.456) (end 115.824 90.932) (width 0.25) (layer "F.Cu") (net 17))
 (segment (start 115.824 90.932) (end 115.824 89.725) (width 0.25) (layer "F.Cu") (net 17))
 (segment (start 127.508 92.456) (end 117.348 92.456) (width 0.25) (layer "F.Cu") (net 17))
 (segment (start 114.3 90.932) (end 114.3 89.725) (width 0.25) (layer "F.Cu") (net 10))
 (segment (start 115.788 110.2) (end 114.3 108.712) (width 0.25) (layer "F.Cu") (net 10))
 (segment (start 128.909 110.2) (end 135.409 110.2) (width 0.25) (layer "F.Cu") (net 10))
 (segment (start 128.909 110.2) (end 115.788 110.2) (width 0.25) (layer "F.Cu") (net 10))
 (via (at 114.3 90.932) (size 0.8) (drill 0.4) (layers "F.Cu" "B.Cu") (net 10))
 (via (at 114.3 108.712) (size 0.8) (drill 0.4) (layers "F.Cu" "B.Cu") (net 10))
 (segment (start 114.174 108.586) (end 114.174 91.058) (width 0.25) (layer "B.Cu") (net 10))
 (segment (start 114.174 91.058) (end 114.3 90.932) (width 0.25) (layer "B.Cu") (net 10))
 (segment (start 114.3 108.712) (end 114.174 108.586) (width 0.25) (layer "B.Cu") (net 10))
 (segment (start 124.765 100.603) (end 113.811 100.603) (width 0.25) (layer "F.Cu") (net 3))
 (segment (start 126.896 100.584) (end 125.84 99.528) (width 0.25) (layer "F.Cu") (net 3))
 (segment (start 137.284 100.584) (end 126.896 100.584) (width 0.25) (layer "F.Cu") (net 3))
 (segment (start 125.84 99.528) (end 124.765 100.603) (width 0.25) (layer "F.Cu") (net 3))
 (segment (start 112.776 90.932) (end 112.776 89.725) (width 0.25) (layer "F.Cu") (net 3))
 (segment (start 138.34 99.528) (end 137.284 100.584) (width 0.25) (layer "F.Cu") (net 3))
 (segment (start 113.811 100.603) (end 112.776 99.568) (width 0.25) (layer "F.Cu") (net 3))
 (via (at 112.776 90.932) (size 0.8) (drill 0.4) (layers "F.Cu" "B.Cu") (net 3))
 (via (at 112.776 99.568) (size 0.8) (drill 0.4) (layers "F.Cu" "B.Cu") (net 3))
 (segment (start 112.776 99.568) (end 112.776 90.932) (width 0.25) (layer "B.Cu") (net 3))
 (segment (start 115.499 94.778) (end 121.999 94.778) (width 0.25) (layer "F.Cu") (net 13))
 (segment (start 121.999 94.778) (end 123.233 96.012) (width 0.25) (layer "F.Cu") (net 13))
 (segment (start 123.233 96.012) (end 135.636 96.012) (width 0.25) (layer "F.Cu") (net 13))
 (via (at 135.636 96.012) (size 0.8) (drill 0.4) (layers "F.Cu" "B.Cu") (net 13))
 (segment (start 135.636 101.6) (end 137.16 103.124) (width 0.25) (layer "B.Cu") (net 13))
 (segment (start 135.636 96.012) (end 135.636 101.6) (width 0.25) (layer "B.Cu") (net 13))
 (segment (start 137.156 103.128) (end 137.156 127) (width 0.25) (layer "B.Cu") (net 13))
 (segment (start 137.16 103.124) (end 137.156 103.128) (width 0.25) (layer "B.Cu") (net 13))
 (segment (start 142.423 94.778) (end 148.923 94.778) (width 0.25) (layer "F.Cu") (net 21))
 (segment (start 128.83 83.602) (end 135.33 83.602) (width 0.25) (layer "F.Cu") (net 16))
 (via (at 133.096 122.936) (size 0.8) (drill 0.4) (layers "F.Cu" "B.Cu") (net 16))
 (segment (start 133.096 85.836) (end 133.096 122.936) (width 0.25) (layer "B.Cu") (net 16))
 (segment (start 135.33 83.602) (end 133.096 85.836) (width 0.25) (layer "B.Cu") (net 16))
 (segment (start 135.409 105.7) (end 128.909 105.7) (width 0.25) (layer "F.Cu") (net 9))
 (segment (start 125.84 94.528) (end 138.34 94.528) (width 0.25) (layer "F.Cu") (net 20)))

